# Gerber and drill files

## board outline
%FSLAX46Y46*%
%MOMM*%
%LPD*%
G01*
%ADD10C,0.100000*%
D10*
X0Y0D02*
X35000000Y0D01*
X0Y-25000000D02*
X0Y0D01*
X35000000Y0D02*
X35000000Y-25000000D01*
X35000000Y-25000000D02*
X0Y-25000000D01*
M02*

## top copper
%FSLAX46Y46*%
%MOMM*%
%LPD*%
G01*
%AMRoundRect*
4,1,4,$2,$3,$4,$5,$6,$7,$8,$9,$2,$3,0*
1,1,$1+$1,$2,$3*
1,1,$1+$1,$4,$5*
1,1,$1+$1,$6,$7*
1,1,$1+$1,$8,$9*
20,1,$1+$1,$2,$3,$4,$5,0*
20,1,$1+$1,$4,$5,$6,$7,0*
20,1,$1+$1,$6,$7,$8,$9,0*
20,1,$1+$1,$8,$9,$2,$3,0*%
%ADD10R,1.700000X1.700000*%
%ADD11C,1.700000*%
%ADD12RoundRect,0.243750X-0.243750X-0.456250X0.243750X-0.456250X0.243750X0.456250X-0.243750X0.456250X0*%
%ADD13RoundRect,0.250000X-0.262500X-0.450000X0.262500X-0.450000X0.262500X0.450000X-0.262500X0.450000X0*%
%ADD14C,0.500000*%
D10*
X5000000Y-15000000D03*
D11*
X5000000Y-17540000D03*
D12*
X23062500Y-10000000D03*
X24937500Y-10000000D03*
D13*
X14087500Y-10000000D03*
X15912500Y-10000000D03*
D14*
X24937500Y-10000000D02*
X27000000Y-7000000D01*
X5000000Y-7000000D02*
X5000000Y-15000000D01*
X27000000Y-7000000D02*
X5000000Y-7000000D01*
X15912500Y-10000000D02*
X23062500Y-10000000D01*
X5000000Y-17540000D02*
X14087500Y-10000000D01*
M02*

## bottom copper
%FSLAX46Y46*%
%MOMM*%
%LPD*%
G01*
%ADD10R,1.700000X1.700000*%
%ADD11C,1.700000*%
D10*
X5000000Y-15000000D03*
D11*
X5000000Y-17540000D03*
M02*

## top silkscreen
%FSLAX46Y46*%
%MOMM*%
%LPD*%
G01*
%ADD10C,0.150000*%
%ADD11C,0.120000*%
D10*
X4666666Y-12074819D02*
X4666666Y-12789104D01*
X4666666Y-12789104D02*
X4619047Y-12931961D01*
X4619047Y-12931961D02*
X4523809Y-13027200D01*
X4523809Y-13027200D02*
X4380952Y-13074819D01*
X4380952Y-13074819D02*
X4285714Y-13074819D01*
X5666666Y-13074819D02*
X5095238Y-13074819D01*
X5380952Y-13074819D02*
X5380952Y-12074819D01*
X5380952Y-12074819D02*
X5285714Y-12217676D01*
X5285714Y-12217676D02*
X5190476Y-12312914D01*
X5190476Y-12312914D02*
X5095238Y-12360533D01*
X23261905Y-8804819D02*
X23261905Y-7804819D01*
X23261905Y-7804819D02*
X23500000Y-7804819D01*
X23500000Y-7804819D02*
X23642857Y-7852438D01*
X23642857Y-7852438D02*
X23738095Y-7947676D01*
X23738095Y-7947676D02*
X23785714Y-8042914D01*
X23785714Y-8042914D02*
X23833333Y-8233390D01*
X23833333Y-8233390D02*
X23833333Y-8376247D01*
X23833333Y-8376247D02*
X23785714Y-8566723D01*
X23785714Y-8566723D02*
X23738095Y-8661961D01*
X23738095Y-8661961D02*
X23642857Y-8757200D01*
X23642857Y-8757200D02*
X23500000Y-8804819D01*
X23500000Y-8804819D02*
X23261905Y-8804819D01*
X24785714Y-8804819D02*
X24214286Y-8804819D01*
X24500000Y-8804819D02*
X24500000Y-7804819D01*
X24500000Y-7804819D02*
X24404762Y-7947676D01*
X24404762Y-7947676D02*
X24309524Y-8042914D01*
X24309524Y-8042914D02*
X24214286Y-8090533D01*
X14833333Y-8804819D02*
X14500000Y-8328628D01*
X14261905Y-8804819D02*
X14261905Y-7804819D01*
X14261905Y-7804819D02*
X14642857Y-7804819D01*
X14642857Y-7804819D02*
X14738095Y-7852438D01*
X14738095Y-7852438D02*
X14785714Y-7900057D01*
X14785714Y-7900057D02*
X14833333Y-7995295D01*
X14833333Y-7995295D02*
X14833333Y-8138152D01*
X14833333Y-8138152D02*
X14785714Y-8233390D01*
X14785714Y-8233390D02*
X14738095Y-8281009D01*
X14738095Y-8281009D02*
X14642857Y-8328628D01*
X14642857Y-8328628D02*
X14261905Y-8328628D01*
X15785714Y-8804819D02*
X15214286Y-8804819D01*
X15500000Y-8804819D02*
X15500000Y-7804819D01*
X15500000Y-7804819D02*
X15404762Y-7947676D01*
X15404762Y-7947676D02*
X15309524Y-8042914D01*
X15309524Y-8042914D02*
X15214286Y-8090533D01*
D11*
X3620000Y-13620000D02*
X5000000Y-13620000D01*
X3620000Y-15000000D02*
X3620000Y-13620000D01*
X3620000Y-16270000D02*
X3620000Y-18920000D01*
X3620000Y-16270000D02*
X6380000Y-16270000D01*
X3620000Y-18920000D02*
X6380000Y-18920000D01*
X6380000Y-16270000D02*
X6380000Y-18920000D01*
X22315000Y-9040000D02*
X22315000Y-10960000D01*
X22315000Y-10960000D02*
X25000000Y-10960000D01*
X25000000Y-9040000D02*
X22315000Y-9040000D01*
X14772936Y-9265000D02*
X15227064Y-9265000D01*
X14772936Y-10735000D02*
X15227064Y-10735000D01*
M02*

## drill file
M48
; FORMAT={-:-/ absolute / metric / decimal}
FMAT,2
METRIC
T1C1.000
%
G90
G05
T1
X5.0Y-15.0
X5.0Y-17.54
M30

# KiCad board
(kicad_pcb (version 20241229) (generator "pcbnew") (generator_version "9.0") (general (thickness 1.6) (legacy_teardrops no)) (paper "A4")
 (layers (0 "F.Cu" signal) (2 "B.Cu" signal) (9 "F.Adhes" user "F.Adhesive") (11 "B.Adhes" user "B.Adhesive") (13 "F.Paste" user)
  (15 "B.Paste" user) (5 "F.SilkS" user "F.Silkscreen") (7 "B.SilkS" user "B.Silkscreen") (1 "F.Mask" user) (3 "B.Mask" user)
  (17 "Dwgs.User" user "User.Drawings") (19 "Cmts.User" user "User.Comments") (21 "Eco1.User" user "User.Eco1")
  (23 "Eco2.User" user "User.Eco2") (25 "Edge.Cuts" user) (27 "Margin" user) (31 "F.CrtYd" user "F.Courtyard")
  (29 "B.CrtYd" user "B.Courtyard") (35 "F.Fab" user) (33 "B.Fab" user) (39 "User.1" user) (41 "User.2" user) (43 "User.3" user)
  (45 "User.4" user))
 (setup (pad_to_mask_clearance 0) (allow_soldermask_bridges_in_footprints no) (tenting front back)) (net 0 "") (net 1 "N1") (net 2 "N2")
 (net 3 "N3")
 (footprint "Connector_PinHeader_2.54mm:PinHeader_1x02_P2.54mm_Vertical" (layer "F.Cu") (at 5 15)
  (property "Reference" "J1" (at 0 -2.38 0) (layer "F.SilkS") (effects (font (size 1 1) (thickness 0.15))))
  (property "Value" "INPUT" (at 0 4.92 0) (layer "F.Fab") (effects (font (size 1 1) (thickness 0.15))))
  (fp_line (start -1.38 -1.38) (end 0 -1.38) (stroke (width 0.12) (type solid)) (layer "F.SilkS"))
  (fp_line (start -1.38 0) (end -1.38 -1.38) (stroke (width 0.12) (type solid)) (layer "F.SilkS"))
  (fp_line (start -1.38 1.27) (end -1.38 3.92) (stroke (width 0.12) (type solid)) (layer "F.SilkS"))
  (fp_line (start -1.38 1.27) (end 1.38 1.27) (stroke (width 0.12) (type solid)) (layer "F.SilkS"))
  (fp_line (start -1.38 3.92) (end 1.38 3.92) (stroke (width 0.12) (type solid)) (layer "F.SilkS"))
  (fp_line (start 1.38 1.27) (end 1.38 3.92) (stroke (width 0.12) (type solid)) (layer "F.SilkS"))
  (pad "1" thru_hole rect (at 0 0) (size 1.7 1.7) (drill 1) (layers "*.Cu" "*.Mask") (remove_unused_layers no) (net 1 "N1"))
  (pad "2" thru_hole circle (at 0 2.54) (size 1.7 1.7) (drill 1) (layers "*.Cu" "*.Mask") (remove_unused_layers no) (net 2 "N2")))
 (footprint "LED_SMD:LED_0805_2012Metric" (layer "F.Cu") (at 24 10)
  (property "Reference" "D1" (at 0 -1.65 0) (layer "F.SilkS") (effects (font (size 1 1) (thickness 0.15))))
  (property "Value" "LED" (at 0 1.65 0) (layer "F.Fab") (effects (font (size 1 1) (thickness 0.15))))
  (fp_line (start -1.685 -0.96) (end -1.685 0.96) (stroke (width 0.12) (type solid)) (layer "F.SilkS"))
  (fp_line (start -1.685 0.96) (end 1 0.96) (stroke (width 0.12) (type solid)) (layer "F.SilkS"))
  (fp_line (start 1 -0.96) (end -1.685 -0.96) (stroke (width 0.12) (type solid)) (layer "F.SilkS"))
  (pad "1" smd roundrect (at -0.9375 0) (size 0.975 1.4) (layers "F.Cu" "F.Mask" "F.Paste") (roundrect_rratio 0.25) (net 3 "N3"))
  (pad "2" smd roundrect (at 0.9375 0) (size 0.975 1.4) (layers "F.Cu" "F.Mask" "F.Paste") (roundrect_rratio 0.25) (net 1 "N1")))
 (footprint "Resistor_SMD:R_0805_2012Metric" (layer "F.Cu") (at 15 10)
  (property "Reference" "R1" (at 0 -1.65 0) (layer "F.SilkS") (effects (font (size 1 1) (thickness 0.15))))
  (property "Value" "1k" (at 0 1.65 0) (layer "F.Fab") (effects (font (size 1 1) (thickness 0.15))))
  (fp_line (start -0.227064 -0.735) (end 0.227064 -0.735) (stroke (width 0.12) (type solid)) (layer "F.SilkS"))
  (fp_line (start -0.227064 0.735) (end 0.227064 0.735) (stroke (width 0.12) (type solid)) (layer "F.SilkS"))
  (pad "1" smd roundrect (at -0.9125 0) (size 1.025 1.4) (layers "F.Cu" "F.Mask" "F.Paste") (roundrect_rratio 0.243902) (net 2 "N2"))
  (pad "2" smd roundrect (at 0.9125 0) (size 1.025 1.4) (layers "F.Cu" "F.Mask" "F.Paste") (roundrect_rratio 0.243902) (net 3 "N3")))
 (gr_line (start 0 0) (end 35 0) (stroke (width 0.1) (type default)) (layer "Edge.Cuts"))
 (gr_line (start 0 25) (end 0 0) (stroke (width 0.1) (type default)) (layer "Edge.Cuts"))
 (gr_line (start 35 0) (end 35 25) (stroke (width 0.1) (type default)) (layer "Edge.Cuts"))
 (gr_line (start 35 25) (end 0 25) (stroke (width 0.1) (type default)) (layer "Edge.Cuts"))
 (segment (start 24.9375 10) (end 27 7) (width 0.5) (layer "F.Cu") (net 1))
 (segment (start 5 7) (end 5 15) (width 0.5) (layer "F.Cu") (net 1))
 (segment (start 27 7) (end 5 7) (width 0.5) (layer "F.Cu") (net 1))
 (segment (start 15.9125 10) (end 23.0625 10) (width 0.5) (layer "F.Cu") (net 3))
 (segment (start 5 17.54) (end 14.0875 10) (width 0.5) (layer "F.Cu") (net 2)))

